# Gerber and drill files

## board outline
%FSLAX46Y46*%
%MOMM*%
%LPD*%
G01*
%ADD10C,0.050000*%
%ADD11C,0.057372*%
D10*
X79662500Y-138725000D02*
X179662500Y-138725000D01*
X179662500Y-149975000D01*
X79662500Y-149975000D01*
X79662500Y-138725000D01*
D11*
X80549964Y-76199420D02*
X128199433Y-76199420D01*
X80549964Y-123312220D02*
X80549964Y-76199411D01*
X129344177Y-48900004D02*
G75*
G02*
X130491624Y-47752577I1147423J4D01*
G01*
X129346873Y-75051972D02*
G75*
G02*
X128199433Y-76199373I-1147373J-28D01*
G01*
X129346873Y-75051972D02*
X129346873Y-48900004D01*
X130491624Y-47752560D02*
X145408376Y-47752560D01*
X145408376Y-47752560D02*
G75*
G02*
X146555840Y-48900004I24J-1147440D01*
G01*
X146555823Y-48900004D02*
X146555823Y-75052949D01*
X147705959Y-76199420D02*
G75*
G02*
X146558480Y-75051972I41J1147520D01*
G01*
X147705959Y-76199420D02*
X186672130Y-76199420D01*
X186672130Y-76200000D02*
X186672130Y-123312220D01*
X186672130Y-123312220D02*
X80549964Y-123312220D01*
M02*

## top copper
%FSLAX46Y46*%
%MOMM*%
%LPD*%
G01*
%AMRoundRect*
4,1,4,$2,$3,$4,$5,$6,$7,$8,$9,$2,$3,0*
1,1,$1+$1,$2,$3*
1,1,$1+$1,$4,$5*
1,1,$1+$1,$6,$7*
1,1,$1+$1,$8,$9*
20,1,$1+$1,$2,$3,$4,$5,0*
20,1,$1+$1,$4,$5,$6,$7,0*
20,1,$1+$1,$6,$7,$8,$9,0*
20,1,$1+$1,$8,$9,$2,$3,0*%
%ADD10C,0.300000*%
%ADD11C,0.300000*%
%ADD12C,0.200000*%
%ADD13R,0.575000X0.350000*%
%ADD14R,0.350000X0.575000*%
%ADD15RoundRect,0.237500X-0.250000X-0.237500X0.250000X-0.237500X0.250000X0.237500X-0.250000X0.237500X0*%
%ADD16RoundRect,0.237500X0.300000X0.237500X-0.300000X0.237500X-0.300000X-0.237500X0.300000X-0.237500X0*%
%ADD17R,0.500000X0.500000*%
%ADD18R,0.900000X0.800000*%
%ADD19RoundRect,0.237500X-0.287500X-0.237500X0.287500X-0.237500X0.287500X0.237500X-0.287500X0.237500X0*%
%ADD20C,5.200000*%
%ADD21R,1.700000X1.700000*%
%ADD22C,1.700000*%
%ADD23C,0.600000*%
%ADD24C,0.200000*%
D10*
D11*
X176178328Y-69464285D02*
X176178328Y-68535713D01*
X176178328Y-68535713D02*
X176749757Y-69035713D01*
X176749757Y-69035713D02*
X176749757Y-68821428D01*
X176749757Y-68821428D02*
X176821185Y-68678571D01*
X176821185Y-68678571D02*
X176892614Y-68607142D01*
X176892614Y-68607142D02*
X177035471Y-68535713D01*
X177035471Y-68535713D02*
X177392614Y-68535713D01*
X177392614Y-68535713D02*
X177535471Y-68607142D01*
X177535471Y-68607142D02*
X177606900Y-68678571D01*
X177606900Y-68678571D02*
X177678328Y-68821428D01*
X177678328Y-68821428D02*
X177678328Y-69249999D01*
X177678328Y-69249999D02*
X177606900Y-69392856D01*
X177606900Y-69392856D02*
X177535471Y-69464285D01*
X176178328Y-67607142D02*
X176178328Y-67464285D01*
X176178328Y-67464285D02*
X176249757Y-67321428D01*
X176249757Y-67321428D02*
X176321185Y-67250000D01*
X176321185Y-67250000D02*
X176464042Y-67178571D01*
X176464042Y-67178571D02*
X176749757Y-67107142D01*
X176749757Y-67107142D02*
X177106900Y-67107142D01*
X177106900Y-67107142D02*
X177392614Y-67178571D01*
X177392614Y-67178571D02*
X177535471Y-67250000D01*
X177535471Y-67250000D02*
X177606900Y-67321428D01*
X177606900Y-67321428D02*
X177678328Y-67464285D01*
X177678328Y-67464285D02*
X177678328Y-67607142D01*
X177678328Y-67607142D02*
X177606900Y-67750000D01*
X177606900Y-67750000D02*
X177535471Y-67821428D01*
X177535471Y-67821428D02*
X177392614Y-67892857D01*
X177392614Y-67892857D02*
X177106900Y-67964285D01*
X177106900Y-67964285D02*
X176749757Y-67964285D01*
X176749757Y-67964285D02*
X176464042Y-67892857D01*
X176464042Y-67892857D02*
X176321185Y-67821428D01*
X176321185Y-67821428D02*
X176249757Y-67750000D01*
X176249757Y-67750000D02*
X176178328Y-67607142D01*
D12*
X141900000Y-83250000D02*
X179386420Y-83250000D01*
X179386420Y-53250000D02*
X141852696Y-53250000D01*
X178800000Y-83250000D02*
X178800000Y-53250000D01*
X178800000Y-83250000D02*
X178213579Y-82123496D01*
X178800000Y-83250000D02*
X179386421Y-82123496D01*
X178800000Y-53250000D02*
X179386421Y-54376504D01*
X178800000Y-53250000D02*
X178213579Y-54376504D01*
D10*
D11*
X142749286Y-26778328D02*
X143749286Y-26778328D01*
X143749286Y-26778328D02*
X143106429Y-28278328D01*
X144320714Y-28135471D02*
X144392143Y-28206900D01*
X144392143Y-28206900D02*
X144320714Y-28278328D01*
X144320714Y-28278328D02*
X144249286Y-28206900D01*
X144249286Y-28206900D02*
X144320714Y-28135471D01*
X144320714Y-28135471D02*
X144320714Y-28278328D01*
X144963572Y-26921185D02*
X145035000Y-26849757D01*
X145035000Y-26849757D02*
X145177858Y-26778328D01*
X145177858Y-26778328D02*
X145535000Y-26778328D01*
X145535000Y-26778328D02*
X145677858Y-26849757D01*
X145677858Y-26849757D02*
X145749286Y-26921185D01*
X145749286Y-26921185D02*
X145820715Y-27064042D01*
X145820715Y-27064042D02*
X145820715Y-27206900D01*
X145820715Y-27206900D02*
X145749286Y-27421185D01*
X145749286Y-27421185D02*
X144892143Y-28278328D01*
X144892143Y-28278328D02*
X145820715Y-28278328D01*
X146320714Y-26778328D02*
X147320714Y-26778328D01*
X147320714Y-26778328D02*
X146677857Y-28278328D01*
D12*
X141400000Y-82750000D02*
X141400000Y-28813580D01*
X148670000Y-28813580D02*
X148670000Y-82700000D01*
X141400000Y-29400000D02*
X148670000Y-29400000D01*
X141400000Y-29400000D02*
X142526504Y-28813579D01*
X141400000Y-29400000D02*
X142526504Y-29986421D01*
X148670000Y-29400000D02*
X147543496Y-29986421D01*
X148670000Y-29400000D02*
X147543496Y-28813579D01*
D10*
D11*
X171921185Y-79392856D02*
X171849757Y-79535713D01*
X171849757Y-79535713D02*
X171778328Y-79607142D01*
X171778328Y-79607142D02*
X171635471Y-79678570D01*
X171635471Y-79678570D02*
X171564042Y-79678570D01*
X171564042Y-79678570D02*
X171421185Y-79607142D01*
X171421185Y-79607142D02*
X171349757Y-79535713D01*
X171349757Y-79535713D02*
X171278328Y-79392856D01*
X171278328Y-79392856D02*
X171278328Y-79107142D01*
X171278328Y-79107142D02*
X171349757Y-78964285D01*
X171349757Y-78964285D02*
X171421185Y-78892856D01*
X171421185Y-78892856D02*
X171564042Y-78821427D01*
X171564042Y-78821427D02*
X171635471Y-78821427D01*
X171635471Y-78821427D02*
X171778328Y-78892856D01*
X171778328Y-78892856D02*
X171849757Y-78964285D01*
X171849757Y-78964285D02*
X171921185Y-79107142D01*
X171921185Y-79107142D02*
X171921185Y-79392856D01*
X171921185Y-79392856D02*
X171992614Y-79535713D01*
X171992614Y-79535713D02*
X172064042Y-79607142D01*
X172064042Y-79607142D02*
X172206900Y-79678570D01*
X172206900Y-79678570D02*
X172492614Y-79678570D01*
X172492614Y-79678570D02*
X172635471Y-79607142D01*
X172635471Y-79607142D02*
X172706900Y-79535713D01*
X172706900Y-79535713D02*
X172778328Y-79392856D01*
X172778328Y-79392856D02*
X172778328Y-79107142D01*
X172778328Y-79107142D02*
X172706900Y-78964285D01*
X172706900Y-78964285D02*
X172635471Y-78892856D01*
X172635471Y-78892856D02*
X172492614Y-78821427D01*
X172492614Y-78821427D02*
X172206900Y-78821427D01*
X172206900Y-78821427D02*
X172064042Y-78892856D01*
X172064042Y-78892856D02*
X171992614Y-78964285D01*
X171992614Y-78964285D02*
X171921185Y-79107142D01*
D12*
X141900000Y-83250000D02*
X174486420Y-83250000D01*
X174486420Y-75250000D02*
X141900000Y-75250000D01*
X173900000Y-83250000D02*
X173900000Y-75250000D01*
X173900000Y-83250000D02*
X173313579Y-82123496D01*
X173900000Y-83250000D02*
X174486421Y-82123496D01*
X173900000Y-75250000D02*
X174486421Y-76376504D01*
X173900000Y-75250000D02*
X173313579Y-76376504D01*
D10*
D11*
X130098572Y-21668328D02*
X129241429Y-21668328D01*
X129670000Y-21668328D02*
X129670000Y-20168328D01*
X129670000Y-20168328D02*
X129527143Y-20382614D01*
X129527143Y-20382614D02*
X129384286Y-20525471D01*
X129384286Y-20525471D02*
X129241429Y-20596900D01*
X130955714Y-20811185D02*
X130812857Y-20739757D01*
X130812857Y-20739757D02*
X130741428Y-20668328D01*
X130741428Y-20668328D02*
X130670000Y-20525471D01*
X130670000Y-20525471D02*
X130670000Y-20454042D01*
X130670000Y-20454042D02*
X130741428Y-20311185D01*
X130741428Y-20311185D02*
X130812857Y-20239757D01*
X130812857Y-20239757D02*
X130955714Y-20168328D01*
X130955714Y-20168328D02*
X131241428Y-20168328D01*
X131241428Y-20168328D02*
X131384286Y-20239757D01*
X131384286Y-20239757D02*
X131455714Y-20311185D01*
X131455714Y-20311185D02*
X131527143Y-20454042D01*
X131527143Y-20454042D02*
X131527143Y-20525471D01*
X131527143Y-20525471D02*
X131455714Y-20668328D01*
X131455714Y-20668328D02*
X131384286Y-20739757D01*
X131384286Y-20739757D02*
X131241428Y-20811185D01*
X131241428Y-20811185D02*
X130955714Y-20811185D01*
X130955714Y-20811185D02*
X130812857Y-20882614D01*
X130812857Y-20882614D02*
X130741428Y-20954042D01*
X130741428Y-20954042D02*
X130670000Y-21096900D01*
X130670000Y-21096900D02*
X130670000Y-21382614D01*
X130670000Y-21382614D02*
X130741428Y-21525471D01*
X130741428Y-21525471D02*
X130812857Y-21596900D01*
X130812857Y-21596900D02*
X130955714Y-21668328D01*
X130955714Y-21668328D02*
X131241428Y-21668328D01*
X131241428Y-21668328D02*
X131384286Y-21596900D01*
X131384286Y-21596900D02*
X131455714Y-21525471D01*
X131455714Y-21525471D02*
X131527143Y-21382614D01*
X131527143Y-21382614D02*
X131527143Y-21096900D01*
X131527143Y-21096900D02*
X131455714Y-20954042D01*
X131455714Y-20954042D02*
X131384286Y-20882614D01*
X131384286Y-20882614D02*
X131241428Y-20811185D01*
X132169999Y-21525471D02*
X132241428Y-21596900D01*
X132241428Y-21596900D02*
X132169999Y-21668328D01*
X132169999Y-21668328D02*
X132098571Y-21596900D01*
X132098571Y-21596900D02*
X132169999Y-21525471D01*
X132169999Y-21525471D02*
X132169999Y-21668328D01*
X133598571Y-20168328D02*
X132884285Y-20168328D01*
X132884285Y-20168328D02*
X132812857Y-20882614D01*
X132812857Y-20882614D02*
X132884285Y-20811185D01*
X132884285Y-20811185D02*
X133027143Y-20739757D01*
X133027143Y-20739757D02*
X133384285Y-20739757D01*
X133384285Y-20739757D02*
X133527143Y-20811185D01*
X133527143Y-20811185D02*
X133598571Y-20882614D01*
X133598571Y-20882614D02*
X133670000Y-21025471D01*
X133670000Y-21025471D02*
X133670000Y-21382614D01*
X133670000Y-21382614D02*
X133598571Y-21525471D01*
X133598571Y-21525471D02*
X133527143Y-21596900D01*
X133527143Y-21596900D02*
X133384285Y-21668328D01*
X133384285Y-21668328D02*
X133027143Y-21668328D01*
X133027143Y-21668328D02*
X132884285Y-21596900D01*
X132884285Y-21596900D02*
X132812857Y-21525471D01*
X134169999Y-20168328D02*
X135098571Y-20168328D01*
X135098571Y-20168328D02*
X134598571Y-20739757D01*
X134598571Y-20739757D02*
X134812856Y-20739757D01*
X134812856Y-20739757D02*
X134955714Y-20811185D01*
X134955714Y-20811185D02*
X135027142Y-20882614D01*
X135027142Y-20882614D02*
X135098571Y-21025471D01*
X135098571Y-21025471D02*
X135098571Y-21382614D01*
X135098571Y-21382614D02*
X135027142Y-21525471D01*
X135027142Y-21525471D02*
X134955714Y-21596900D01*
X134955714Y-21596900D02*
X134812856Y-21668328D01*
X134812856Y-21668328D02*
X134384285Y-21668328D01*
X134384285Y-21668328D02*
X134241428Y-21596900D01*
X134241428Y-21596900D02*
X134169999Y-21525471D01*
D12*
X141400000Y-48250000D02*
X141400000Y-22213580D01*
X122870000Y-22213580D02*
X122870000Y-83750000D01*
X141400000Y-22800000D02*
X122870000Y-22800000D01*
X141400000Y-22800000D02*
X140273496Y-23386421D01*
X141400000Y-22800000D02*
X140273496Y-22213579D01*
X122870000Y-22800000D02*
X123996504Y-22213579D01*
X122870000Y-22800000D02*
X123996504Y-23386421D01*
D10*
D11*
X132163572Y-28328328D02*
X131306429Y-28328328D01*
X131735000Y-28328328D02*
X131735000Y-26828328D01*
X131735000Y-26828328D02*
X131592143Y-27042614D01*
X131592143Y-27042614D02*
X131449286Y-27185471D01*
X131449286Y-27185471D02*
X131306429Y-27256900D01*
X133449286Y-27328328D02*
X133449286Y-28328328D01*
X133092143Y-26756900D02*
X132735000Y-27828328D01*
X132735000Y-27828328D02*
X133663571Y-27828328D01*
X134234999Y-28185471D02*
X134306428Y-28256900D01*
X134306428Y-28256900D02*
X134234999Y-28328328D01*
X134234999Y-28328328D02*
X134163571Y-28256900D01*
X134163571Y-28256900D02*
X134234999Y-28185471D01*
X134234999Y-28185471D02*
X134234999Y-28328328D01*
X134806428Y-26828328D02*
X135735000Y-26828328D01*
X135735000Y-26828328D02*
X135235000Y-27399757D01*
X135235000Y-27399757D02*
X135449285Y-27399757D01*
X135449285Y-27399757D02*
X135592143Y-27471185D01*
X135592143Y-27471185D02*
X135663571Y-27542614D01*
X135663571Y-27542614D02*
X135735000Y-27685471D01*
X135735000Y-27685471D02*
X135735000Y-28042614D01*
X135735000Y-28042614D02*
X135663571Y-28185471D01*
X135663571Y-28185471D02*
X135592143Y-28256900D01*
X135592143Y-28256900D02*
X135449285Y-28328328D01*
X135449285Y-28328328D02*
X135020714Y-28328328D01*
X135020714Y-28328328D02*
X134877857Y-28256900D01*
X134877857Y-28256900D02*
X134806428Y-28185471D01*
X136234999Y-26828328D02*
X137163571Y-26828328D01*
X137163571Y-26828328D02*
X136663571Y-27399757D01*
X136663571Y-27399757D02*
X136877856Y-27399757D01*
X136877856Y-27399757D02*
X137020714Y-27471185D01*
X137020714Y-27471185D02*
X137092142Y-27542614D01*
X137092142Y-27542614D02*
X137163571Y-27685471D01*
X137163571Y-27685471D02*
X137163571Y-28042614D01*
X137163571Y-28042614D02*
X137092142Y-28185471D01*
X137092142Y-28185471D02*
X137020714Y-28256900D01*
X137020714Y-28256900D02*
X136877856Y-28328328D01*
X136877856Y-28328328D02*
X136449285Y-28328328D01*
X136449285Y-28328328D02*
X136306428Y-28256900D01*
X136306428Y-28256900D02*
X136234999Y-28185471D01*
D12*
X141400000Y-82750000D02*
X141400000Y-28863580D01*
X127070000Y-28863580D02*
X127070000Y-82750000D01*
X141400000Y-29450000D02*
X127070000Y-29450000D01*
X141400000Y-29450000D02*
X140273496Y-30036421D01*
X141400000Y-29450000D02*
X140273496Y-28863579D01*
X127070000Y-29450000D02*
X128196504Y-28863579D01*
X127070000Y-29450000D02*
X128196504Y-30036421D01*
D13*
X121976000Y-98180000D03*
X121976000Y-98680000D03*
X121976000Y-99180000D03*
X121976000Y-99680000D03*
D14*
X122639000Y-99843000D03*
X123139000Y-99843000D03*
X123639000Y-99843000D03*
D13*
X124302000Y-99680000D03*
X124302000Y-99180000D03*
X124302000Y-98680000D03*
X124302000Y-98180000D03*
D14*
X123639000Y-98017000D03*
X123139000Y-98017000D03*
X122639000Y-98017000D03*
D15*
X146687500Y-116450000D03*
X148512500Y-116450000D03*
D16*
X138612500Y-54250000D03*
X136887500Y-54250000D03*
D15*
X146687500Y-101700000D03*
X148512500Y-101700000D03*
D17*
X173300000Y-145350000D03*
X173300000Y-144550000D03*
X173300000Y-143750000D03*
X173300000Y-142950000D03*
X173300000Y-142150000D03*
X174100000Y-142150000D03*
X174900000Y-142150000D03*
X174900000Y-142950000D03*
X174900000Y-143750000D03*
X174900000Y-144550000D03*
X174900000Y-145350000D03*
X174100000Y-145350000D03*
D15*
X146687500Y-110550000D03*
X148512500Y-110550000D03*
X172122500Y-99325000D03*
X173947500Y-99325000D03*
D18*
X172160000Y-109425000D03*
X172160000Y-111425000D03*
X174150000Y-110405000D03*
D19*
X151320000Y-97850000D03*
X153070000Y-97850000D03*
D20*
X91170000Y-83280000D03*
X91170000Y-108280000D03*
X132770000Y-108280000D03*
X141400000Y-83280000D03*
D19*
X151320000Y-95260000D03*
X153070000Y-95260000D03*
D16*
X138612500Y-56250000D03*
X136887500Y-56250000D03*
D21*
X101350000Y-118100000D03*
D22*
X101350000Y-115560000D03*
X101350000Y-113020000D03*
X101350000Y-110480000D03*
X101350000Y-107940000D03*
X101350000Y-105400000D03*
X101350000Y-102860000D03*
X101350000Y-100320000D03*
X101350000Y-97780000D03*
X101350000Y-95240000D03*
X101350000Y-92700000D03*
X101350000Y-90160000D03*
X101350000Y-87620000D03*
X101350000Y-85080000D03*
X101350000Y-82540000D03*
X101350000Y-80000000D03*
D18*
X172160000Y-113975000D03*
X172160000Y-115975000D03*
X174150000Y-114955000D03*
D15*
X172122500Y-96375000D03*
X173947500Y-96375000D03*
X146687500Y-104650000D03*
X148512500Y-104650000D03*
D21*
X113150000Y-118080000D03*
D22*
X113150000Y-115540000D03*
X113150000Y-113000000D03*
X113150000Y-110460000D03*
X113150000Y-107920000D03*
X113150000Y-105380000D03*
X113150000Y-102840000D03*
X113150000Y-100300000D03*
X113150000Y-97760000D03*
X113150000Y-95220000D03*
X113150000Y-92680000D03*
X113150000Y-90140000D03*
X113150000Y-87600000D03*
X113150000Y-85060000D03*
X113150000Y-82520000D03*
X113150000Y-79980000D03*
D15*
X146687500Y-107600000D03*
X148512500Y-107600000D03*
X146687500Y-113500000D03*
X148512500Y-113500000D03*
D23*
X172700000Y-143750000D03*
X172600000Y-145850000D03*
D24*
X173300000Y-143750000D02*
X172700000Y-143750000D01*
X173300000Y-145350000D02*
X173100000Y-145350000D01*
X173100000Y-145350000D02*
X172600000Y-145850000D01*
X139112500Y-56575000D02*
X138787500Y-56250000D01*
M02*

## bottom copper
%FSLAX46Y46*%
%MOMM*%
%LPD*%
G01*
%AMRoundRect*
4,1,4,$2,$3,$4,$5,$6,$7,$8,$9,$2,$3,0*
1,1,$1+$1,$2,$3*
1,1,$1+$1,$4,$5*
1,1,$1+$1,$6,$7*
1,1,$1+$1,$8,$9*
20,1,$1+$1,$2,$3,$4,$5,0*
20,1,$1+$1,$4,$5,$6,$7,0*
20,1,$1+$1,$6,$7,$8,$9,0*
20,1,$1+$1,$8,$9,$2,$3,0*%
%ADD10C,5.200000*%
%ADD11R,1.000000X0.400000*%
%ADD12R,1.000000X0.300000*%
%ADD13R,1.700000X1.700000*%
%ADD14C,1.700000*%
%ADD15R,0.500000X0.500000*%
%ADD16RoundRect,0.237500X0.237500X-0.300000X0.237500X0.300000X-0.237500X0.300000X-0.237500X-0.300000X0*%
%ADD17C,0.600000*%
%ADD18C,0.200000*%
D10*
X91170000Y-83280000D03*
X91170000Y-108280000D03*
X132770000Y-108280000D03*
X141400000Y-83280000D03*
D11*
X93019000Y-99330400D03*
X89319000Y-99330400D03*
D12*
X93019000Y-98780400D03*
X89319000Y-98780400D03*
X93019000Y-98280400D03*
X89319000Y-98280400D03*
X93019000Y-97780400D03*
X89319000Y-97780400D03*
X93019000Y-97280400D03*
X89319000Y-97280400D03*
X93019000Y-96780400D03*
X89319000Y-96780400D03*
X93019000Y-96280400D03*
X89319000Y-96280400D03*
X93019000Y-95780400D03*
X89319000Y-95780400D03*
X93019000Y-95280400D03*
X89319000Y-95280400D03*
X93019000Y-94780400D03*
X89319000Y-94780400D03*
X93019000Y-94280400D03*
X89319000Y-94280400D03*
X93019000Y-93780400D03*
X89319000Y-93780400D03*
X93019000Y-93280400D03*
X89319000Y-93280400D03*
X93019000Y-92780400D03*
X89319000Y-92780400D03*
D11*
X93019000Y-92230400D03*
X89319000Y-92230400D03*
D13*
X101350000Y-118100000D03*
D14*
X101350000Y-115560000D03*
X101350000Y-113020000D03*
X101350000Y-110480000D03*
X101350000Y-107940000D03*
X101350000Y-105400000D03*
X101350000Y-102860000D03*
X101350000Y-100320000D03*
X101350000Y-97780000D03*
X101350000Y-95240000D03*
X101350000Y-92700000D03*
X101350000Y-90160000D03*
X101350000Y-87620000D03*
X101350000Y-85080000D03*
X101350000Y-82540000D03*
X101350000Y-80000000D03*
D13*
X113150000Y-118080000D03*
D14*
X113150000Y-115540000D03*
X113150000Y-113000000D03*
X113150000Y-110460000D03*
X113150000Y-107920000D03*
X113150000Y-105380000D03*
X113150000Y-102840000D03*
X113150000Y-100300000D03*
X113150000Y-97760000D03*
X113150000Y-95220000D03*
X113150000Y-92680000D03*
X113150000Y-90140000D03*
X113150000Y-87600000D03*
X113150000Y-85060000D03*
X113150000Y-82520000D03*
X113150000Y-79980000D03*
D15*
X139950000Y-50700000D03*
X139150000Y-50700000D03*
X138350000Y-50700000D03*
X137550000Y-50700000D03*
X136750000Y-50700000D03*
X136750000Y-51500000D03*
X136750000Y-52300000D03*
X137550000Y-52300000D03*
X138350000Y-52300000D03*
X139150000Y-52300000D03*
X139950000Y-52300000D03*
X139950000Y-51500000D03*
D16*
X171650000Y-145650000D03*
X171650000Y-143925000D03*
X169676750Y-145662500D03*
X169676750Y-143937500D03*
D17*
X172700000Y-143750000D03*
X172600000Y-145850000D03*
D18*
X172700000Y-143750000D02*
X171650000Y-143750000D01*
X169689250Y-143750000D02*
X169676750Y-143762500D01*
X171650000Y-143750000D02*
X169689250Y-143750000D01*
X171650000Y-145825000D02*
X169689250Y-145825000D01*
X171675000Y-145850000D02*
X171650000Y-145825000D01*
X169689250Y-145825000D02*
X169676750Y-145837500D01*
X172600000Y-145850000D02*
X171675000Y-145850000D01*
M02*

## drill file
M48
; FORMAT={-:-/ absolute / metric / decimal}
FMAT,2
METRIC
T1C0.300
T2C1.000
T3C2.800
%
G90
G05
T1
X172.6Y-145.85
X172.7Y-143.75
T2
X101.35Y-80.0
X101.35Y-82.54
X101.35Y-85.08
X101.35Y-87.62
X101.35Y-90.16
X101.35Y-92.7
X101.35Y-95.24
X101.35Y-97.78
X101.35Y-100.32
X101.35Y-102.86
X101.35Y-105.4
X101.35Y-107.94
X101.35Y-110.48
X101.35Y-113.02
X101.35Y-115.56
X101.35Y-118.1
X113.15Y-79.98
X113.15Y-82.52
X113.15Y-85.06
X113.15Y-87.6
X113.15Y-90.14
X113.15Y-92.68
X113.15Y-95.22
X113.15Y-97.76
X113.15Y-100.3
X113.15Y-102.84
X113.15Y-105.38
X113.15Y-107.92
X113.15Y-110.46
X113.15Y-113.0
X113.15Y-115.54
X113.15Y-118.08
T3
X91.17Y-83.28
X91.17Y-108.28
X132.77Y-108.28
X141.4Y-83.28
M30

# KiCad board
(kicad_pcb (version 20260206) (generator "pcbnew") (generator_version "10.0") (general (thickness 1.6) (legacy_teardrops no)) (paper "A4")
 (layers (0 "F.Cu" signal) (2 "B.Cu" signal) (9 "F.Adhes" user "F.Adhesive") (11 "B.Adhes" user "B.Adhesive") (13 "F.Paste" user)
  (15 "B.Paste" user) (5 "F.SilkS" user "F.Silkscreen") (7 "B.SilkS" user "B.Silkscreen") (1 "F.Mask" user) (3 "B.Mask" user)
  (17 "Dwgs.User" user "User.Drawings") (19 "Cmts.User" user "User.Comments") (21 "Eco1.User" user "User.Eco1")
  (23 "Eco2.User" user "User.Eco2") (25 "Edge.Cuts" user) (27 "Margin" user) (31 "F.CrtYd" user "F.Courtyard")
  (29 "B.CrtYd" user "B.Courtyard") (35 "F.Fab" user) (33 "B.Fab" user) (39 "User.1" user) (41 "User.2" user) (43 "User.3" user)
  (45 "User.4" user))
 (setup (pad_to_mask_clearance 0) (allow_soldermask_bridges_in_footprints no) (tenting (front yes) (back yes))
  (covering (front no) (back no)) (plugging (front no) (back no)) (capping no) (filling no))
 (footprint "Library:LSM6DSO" (layer "F.Cu") (at 123.139 98.93)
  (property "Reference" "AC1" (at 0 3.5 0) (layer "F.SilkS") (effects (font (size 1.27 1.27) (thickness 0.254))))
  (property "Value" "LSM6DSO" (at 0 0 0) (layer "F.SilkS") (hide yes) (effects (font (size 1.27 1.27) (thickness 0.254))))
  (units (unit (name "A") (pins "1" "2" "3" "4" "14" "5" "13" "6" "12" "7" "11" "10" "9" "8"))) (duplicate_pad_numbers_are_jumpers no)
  (pad "1" smd rect (at -1.163 -0.75 90) (size 0.35 0.575) (layers "F.Cu" "F.Mask" "F.Paste") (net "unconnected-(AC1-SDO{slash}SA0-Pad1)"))
  (pad "2" smd rect (at -1.163 -0.25 90) (size 0.35 0.575) (layers "F.Cu" "F.Mask" "F.Paste") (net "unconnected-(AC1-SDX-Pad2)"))
  (pad "3" smd rect (at -1.163 0.25 90) (size 0.35 0.575) (layers "F.Cu" "F.Mask" "F.Paste") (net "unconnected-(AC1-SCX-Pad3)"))
  (pad "4" smd rect (at -1.163 0.75 90) (size 0.35 0.575) (layers "F.Cu" "F.Mask" "F.Paste") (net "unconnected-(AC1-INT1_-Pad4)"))
  (pad "5" smd rect (at -0.5 0.913) (size 0.35 0.575) (layers "F.Cu" "F.Mask" "F.Paste") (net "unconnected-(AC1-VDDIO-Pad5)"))
  (pad "6" smd rect (at 0 0.913) (size 0.35 0.575) (layers "F.Cu" "F.Mask" "F.Paste") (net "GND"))
  (pad "7" smd rect (at 0.5 0.913) (size 0.35 0.575) (layers "F.Cu" "F.Mask" "F.Paste") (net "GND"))
  (pad "8" smd rect (at 1.163 0.75 90) (size 0.35 0.575) (layers "F.Cu" "F.Mask" "F.Paste") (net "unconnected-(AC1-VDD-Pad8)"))
  (pad "9" smd rect (at 1.163 0.25 90) (size 0.35 0.575) (layers "F.Cu" "F.Mask" "F.Paste") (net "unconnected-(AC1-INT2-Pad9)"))
  (pad "10" smd rect (at 1.163 -0.25 90) (size 0.35 0.575) (layers "F.Cu" "F.Mask" "F.Paste") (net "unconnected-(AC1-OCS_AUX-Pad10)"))
  (pad "11" smd rect (at 1.163 -0.75 90) (size 0.35 0.575) (layers "F.Cu" "F.Mask" "F.Paste") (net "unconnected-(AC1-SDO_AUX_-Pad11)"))
  (pad "12" smd rect (at 0.5 -0.913) (size 0.35 0.575) (layers "F.Cu" "F.Mask" "F.Paste") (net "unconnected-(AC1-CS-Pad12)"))
  (pad "13" smd rect (at 0 -0.913) (size 0.35 0.575) (layers "F.Cu" "F.Mask" "F.Paste") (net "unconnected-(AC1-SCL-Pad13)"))
  (pad "14" smd rect (at -0.5 -0.913) (size 0.35 0.575) (layers "F.Cu" "F.Mask" "F.Paste") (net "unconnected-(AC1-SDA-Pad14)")))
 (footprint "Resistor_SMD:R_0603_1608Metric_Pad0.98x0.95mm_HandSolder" (layer "F.Cu") (at 147.6 116.45)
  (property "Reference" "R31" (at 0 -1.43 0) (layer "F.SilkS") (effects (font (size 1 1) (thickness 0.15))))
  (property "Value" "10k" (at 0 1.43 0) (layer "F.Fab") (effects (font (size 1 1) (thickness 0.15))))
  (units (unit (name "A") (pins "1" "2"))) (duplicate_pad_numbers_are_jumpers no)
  (pad "1" smd roundrect (at -0.9125 0) (size 0.975 0.95) (layers "F.Cu" "F.Mask" "F.Paste") (roundrect_rratio 0.25) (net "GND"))
  (pad "2" smd roundrect (at 0.9125 0) (size 0.975 0.95) (layers "F.Cu" "F.Mask" "F.Paste") (roundrect_rratio 0.25) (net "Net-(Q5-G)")))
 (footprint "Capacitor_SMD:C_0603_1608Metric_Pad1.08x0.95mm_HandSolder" (layer "F.Cu") (at 137.75 54.25 180)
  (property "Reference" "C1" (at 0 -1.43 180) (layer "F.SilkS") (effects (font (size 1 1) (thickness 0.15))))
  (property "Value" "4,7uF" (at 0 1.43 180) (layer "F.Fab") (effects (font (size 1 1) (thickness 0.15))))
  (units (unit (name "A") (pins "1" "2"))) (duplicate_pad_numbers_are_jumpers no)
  (pad "1" smd roundrect (at -0.8625 0 180) (size 1.075 0.95) (layers "F.Cu" "F.Mask" "F.Paste") (roundrect_rratio 0.25) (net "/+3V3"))
  (pad "2" smd roundrect (at 0.8625 0 180) (size 1.075 0.95) (layers "F.Cu" "F.Mask" "F.Paste") (roundrect_rratio 0.25) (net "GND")))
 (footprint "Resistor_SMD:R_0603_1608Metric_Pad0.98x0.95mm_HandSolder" (layer "F.Cu") (at 147.6 101.7)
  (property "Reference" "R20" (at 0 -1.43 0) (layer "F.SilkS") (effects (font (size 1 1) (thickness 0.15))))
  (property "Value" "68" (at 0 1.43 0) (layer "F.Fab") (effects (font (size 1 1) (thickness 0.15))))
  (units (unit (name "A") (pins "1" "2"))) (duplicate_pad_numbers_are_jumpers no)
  (pad "1" smd roundrect (at -0.9125 0) (size 0.975 0.95) (layers "F.Cu" "F.Mask" "F.Paste") (roundrect_rratio 0.25) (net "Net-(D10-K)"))
  (pad "2" smd roundrect (at 0.9125 0) (size 0.975 0.95) (layers "F.Cu" "F.Mask" "F.Paste") (roundrect_rratio 0.25) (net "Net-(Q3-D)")))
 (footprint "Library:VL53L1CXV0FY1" (layer "F.Cu") (at 174.1 143.75 90)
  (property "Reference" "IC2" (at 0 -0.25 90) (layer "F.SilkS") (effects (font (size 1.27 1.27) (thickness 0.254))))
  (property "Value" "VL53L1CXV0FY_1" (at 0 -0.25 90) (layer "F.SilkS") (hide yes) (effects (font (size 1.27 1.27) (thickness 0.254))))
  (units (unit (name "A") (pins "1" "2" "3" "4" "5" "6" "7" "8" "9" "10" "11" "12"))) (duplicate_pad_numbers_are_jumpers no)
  (pad "1" smd rect (at -1.6 -0.8 180) (size 0.5 0.5) (layers "F.Cu" "F.Mask" "F.Paste") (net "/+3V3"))
  (pad "2" smd rect (at -0.8 -0.8 180) (size 0.5 0.5) (layers "F.Cu" "F.Mask" "F.Paste") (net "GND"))
  (pad "3" smd rect (at 0 -0.8 180) (size 0.5 0.5) (layers "F.Cu" "F.Mask" "F.Paste") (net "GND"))
  (pad "4" smd rect (at 0.8 -0.8 180) (size 0.5 0.5) (layers "F.Cu" "F.Mask" "F.Paste") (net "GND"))
  (pad "5" smd rect (at 1.6 -0.8 180) (size 0.5 0.5) (layers "F.Cu" "F.Mask" "F.Paste") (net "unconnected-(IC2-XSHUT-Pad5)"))
  (pad "6" smd rect (at 1.6 0 180) (size 0.5 0.5) (layers "F.Cu" "F.Mask" "F.Paste") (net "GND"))
  (pad "7" smd rect (at 1.6 0.8 180) (size 0.5 0.5) (layers "F.Cu" "F.Mask" "F.Paste") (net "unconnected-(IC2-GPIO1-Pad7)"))
  (pad "8" smd rect (at 0.8 0.8 180) (size 0.5 0.5) (layers "F.Cu" "F.Mask" "F.Paste") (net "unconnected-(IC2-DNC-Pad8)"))
  (pad "9" smd rect (at 0 0.8 180) (size 0.5 0.5) (layers "F.Cu" "F.Mask" "F.Paste") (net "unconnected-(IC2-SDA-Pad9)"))
  (pad "10" smd rect (at -0.8 0.8 180) (size 0.5 0.5) (layers "F.Cu" "F.Mask" "F.Paste") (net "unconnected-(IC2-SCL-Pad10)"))
  (pad "11" smd rect (at -1.6 0.8 180) (size 0.5 0.5) (layers "F.Cu" "F.Mask" "F.Paste") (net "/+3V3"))
  (pad "12" smd rect (at -1.6 0 180) (size 0.5 0.5) (layers "F.Cu" "F.Mask" "F.Paste") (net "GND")))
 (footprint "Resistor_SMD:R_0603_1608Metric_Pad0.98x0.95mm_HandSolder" (layer "F.Cu") (at 147.6 110.55)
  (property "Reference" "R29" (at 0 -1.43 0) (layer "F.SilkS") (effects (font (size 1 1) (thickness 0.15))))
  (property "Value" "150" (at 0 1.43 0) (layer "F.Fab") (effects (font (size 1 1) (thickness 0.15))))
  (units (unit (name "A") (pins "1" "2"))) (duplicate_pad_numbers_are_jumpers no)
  (pad "1" smd roundrect (at -0.9125 0) (size 0.975 0.95) (layers "F.Cu" "F.Mask" "F.Paste") (roundrect_rratio 0.25) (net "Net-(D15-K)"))
  (pad "2" smd roundrect (at 0.9125 0) (size 0.975 0.95) (layers "F.Cu" "F.Mask" "F.Paste") (roundrect_rratio 0.25) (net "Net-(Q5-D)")))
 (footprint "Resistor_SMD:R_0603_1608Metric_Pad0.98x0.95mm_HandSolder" (layer "F.Cu") (at 173.035 99.325)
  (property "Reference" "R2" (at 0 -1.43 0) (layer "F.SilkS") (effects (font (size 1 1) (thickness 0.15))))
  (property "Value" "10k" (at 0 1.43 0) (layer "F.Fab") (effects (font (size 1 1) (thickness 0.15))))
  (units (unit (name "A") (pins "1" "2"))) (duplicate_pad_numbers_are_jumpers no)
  (pad "1" smd roundrect (at -0.9125 0) (size 0.975 0.95) (layers "F.Cu" "F.Mask" "F.Paste") (roundrect_rratio 0.25)
   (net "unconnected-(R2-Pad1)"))
  (pad "2" smd roundrect (at 0.9125 0) (size 0.975 0.95) (layers "F.Cu" "F.Mask" "F.Paste") (roundrect_rratio 0.25)
   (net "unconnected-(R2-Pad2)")))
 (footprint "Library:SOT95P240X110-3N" (layer "F.Cu") (at 173.15 110.425)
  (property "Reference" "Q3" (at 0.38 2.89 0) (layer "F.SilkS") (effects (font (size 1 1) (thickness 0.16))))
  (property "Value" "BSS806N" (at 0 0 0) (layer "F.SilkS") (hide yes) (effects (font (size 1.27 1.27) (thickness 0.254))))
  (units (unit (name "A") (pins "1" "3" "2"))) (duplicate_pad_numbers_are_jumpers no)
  (pad "1" smd rect (at -0.99 -1) (size 0.9 0.8) (layers "F.Cu" "F.Mask" "F.Paste") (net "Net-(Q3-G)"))
  (pad "2" smd rect (at -0.99 1) (size 0.9 0.8) (layers "F.Cu" "F.Mask" "F.Paste") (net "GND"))
  (pad "3" smd rect (at 1 -0.02) (size 0.9 0.8) (layers "F.Cu" "F.Mask" "F.Paste") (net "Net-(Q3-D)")))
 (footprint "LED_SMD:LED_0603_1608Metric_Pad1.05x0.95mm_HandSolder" (layer "F.Cu") (at 152.195 97.85)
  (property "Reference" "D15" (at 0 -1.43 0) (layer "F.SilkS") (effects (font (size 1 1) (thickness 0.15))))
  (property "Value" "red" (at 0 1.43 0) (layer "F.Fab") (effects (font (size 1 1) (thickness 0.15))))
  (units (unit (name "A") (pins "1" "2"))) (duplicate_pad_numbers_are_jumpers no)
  (pad "1" smd roundrect (at -0.875 0) (size 1.05 0.95) (layers "F.Cu" "F.Mask" "F.Paste") (roundrect_rratio 0.25) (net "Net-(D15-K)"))
  (pad "2" smd roundrect (at 0.875 0) (size 1.05 0.95) (layers "F.Cu" "F.Mask" "F.Paste") (roundrect_rratio 0.25) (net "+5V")))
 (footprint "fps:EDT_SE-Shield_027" (layer "F.Cu") (at 91.17 108.28)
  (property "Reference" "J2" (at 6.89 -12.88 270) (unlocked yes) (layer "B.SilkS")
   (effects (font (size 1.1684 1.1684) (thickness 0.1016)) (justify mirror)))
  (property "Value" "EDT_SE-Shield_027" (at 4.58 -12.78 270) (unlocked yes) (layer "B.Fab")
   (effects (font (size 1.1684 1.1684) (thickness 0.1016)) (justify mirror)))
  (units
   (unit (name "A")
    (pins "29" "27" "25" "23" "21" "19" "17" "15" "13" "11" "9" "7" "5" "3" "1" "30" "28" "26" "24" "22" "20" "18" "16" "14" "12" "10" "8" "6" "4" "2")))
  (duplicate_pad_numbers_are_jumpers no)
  (pad "" thru_hole circle (at 0 -25) (size 5.2 5.2) (drill 2.8) (layers "*.Cu" "*.Mask") (remove_unused_layers no))
  (pad "" thru_hole circle (at 0 0) (size 5.2 5.2) (drill 2.8) (layers "*.Cu" "*.Mask") (remove_unused_layers no))
  (pad "" thru_hole circle (at 41.6 0) (size 5.2 5.2) (drill 2.8) (layers "*.Cu" "*.Mask") (remove_unused_layers no))
  (pad "" thru_hole circle (at 50.23 -25) (size 5.2 5.2) (drill 2.8) (layers "*.Cu" "*.Mask") (remove_unused_layers no))
  (pad "1" smd rect (at 1.849 -8.9496 180) (size 1 0.4) (layers "B.Cu" "B.Mask" "B.Paste") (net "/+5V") (solder_mask_margin 0.075)
   (solder_paste_margin 0) (thermal_bridge_angle 0))
  (pad "2" smd rect (at -1.851 -8.9496 180) (size 1 0.4) (layers "B.Cu" "B.Mask" "B.Paste") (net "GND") (solder_mask_margin 0.075)
   (solder_paste_margin 0) (thermal_bridge_angle 0))
  (pad "3" smd rect (at 1.849 -9.4996 180) (size 1 0.3) (layers "B.Cu" "B.Mask" "B.Paste") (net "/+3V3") (solder_mask_margin 0.075)
   (solder_paste_margin 0) (thermal_bridge_angle 0))
  (pad "4" smd rect (at -1.851 -9.4996 180) (size 1 0.3) (layers "B.Cu" "B.Mask" "B.Paste") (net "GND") (solder_mask_margin 0.075)
   (solder_paste_margin 0) (thermal_bridge_angle 0))
  (pad "5" smd rect (at 1.849 -9.9996 180) (size 1 0.3) (layers "B.Cu" "B.Mask" "B.Paste") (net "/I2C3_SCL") (solder_mask_margin 0.075)
   (solder_paste_margin 0) (thermal_bridge_angle 0))
  (pad "6" smd rect (at -1.851 -9.9996 180) (size 1 0.3) (layers "B.Cu" "B.Mask" "B.Paste") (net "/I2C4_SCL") (solder_mask_margin 0.075)
   (solder_paste_margin 0) (thermal_bridge_angle 0))
  (pad "7" smd rect (at 1.849 -10.4996 180) (size 1 0.3) (layers "B.Cu" "B.Mask" "B.Paste") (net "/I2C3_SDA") (solder_mask_margin 0.075)
   (solder_paste_margin 0) (thermal_bridge_angle 0))
  (pad "8" smd rect (at -1.851 -10.4996 180) (size 1 0.3) (layers "B.Cu" "B.Mask" "B.Paste") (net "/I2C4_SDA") (solder_mask_margin 0.075)
   (solder_paste_margin 0) (thermal_bridge_angle 0))
  (pad "9" smd rect (at 1.849 -10.9996 180) (size 1 0.3) (layers "B.Cu" "B.Mask" "B.Paste") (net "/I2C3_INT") (solder_mask_margin 0.075)
   (solder_paste_margin 0) (thermal_bridge_angle 0))
  (pad "10" smd rect (at -1.851 -10.9996 180) (size 1 0.3) (layers "B.Cu" "B.Mask" "B.Paste") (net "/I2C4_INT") (solder_mask_margin 0.075)
   (solder_paste_margin 0) (thermal_bridge_angle 0))
  (pad "11" smd rect (at 1.849 -11.4996 180) (size 1 0.3) (layers "B.Cu" "B.Mask" "B.Paste") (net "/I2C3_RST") (solder_mask_margin 0.075)
   (solder_paste_margin 0) (thermal_bridge_angle 0))
  (pad "12" smd rect (at -1.851 -11.4996 180) (size 1 0.3) (layers "B.Cu" "B.Mask" "B.Paste") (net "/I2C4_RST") (solder_mask_margin 0.075)
   (solder_paste_margin 0) (thermal_bridge_angle 0))
  (pad "13" smd rect (at 1.849 -11.9996 180) (size 1 0.3) (layers "B.Cu" "B.Mask" "B.Paste") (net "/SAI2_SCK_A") (solder_mask_margin 0.075)
   (solder_paste_margin 0) (thermal_bridge_angle 0))
  (pad "14" smd rect (at -1.851 -11.9996 180) (size 1 0.3) (layers "B.Cu" "B.Mask" "B.Paste") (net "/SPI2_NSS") (solder_mask_margin 0.075)
   (solder_paste_margin 0) (thermal_bridge_angle 0))
  (pad "15" smd rect (at 1.849 -12.4996 180) (size 1 0.3) (layers "B.Cu" "B.Mask" "B.Paste") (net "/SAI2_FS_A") (solder_mask_margin 0.075)
   (solder_paste_margin 0) (thermal_bridge_angle 0))
  (pad "16" smd rect (at -1.851 -12.4996 180) (size 1 0.3) (layers "B.Cu" "B.Mask" "B.Paste") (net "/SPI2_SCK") (solder_mask_margin 0.075)
   (solder_paste_margin 0) (thermal_bridge_angle 0))
  (pad "17" smd rect (at 1.849 -12.9996 180) (size 1 0.3) (layers "B.Cu" "B.Mask" "B.Paste") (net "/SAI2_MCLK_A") (solder_mask_margin 0.075)
   (solder_paste_margin 0) (thermal_bridge_angle 0))
  (pad "18" smd rect (at -1.851 -12.9996 180) (size 1 0.3) (layers "B.Cu" "B.Mask" "B.Paste") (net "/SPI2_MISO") (solder_mask_margin 0.075)
   (solder_paste_margin 0) (thermal_bridge_angle 0))
  (pad "19" smd rect (at 1.849 -13.4996 180) (size 1 0.3) (layers "B.Cu" "B.Mask" "B.Paste") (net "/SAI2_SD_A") (solder_mask_margin 0.075)
   (solder_paste_margin 0) (thermal_bridge_angle 0))
  (pad "20" smd rect (at -1.851 -13.4996 180) (size 1 0.3) (layers "B.Cu" "B.Mask" "B.Paste") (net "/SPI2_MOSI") (solder_mask_margin 0.075)
   (solder_paste_margin 0) (thermal_bridge_angle 0))
  (pad "21" smd rect (at 1.849 -13.9996 180) (size 1 0.3) (layers "B.Cu" "B.Mask" "B.Paste") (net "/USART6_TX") (solder_mask_margin 0.075)
   (solder_paste_margin 0) (thermal_bridge_angle 0))
  (pad "22" smd rect (at -1.851 -13.9996 180) (size 1 0.3) (layers "B.Cu" "B.Mask" "B.Paste") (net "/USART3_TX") (solder_mask_margin 0.075)
   (solder_paste_margin 0) (thermal_bridge_angle 0))
  (pad "23" smd rect (at 1.849 -14.4996 180) (size 1 0.3) (layers "B.Cu" "B.Mask" "B.Paste") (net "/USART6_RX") (solder_mask_margin 0.075)
   (solder_paste_margin 0) (thermal_bridge_angle 0))
  (pad "24" smd rect (at -1.851 -14.4996 180) (size 1 0.3) (layers "B.Cu" "B.Mask" "B.Paste") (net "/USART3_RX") (solder_mask_margin 0.075)
   (solder_paste_margin 0) (thermal_bridge_angle 0))
  (pad "25" smd rect (at 1.849 -14.9996 180) (size 1 0.3) (layers "B.Cu" "B.Mask" "B.Paste") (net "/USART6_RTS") (solder_mask_margin 0.075)
   (solder_paste_margin 0) (thermal_bridge_angle 0))
  (pad "26" smd rect (at -1.851 -14.9996 180) (size 1 0.3) (layers "B.Cu" "B.Mask" "B.Paste") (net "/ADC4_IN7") (solder_mask_margin 0.075)
   (solder_paste_margin 0) (thermal_bridge_angle 0))
  (pad "27" smd rect (at 1.849 -15.4996 180) (size 1 0.3) (layers "B.Cu" "B.Mask" "B.Paste") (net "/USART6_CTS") (solder_mask_margin 0.075)
   (solder_paste_margin 0) (thermal_bridge_angle 0))
  (pad "28" smd rect (at -1.851 -15.4996 180) (size 1 0.3) (layers "B.Cu" "B.Mask" "B.Paste") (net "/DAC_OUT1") (solder_mask_margin 0.075)
   (solder_paste_margin 0) (thermal_bridge_angle 0))
  (pad "29" smd rect (at 1.849 -16.0496 180) (size 1 0.4) (layers "B.Cu" "B.Mask" "B.Paste") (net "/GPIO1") (solder_mask_margin 0.075)
   (solder_paste_margin 0) (thermal_bridge_angle 0))
  (pad "30" smd rect (at -1.851 -16.0496 180) (size 1 0.4) (layers "B.Cu" "B.Mask" "B.Paste") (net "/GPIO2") (solder_mask_margin 0.075)
   (solder_paste_margin 0) (thermal_bridge_angle 0)))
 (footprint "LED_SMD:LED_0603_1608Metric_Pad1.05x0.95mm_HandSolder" (layer "F.Cu") (at 152.195 95.26)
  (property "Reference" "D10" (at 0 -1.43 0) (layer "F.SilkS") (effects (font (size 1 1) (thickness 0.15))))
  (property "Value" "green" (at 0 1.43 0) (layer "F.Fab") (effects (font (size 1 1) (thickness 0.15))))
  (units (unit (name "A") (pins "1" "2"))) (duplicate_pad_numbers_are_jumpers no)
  (pad "1" smd roundrect (at -0.875 0) (size 1.05 0.95) (layers "F.Cu" "F.Mask" "F.Paste") (roundrect_rratio 0.25) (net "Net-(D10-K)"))
  (pad "2" smd roundrect (at 0.875 0) (size 1.05 0.95) (layers "F.Cu" "F.Mask" "F.Paste") (roundrect_rratio 0.25) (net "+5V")))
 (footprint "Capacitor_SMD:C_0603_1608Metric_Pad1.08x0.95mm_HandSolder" (layer "F.Cu") (at 137.75 56.25 180)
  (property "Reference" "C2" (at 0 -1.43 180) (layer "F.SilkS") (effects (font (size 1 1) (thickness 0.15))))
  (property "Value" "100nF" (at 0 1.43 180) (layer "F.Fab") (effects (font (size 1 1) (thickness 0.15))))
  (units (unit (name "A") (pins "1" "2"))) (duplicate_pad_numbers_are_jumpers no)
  (pad "1" smd roundrect (at -0.8625 0 180) (size 1.075 0.95) (layers "F.Cu" "F.Mask" "F.Paste") (roundrect_rratio 0.25) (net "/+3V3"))
  (pad "2" smd roundrect (at 0.8625 0 180) (size 1.075 0.95) (layers "F.Cu" "F.Mask" "F.Paste") (roundrect_rratio 0.25) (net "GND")))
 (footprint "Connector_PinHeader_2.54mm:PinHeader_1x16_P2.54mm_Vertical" (layer "F.Cu") (at 101.35 118.1 180)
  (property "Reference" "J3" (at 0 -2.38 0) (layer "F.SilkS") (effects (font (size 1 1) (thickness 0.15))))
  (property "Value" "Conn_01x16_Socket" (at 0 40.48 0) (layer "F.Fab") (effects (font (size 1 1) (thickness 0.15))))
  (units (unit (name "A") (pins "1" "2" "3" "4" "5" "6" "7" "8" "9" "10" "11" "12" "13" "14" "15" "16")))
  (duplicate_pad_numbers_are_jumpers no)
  (pad "1" thru_hole rect (at 0 0 180) (size 1.7 1.7) (drill 1) (layers "*.Cu" "*.Mask") (remove_unused_layers no) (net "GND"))
  (pad "2" thru_hole circle (at 0 2.54 180) (size 1.7 1.7) (drill 1) (layers "*.Cu" "*.Mask") (remove_unused_layers no) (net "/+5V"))
  (pad "3" thru_hole circle (at 0 5.08 180) (size 1.7 1.7) (drill 1) (layers "*.Cu" "*.Mask") (remove_unused_layers no) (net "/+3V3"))
  (pad "4" thru_hole circle (at 0 7.62 180) (size 1.7 1.7) (drill 1) (layers "*.Cu" "*.Mask") (remove_unused_layers no) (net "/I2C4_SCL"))
  (pad "5" thru_hole circle (at 0 10.16 180) (size 1.7 1.7) (drill 1) (layers "*.Cu" "*.Mask") (remove_unused_layers no) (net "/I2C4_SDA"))
  (pad "6" thru_hole circle (at 0 12.7 180) (size 1.7 1.7) (drill 1) (layers "*.Cu" "*.Mask") (remove_unused_layers no) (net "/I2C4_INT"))
  (pad "7" thru_hole circle (at 0 15.24 180) (size 1.7 1.7) (drill 1) (layers "*.Cu" "*.Mask") (remove_unused_layers no) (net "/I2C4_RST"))
  (pad "8" thru_hole circle (at 0 17.78 180) (size 1.7 1.7) (drill 1) (layers "*.Cu" "*.Mask") (remove_unused_layers no) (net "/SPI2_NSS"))
  (pad "9" thru_hole circle (at 0 20.32 180) (size 1.7 1.7) (drill 1) (layers "*.Cu" "*.Mask") (remove_unused_layers no) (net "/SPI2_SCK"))
  (pad "10" thru_hole circle (at 0 22.86 180) (size 1.7 1.7) (drill 1) (layers "*.Cu" "*.Mask") (remove_unused_layers no) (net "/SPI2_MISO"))
  (pad "11" thru_hole circle (at 0 25.4 180) (size 1.7 1.7) (drill 1) (layers "*.Cu" "*.Mask") (remove_unused_layers no) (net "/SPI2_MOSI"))
  (pad "12" thru_hole circle (at 0 27.94 180) (size 1.7 1.7) (drill 1) (layers "*.Cu" "*.Mask") (remove_unused_layers no) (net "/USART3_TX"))
  (pad "13" thru_hole circle (at 0 30.48 180) (size 1.7 1.7) (drill 1) (layers "*.Cu" "*.Mask") (remove_unused_layers no) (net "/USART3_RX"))
  (pad "14" thru_hole circle (at 0 33.02 180) (size 1.7 1.7) (drill 1) (layers "*.Cu" "*.Mask") (remove_unused_layers no) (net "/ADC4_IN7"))
  (pad "15" thru_hole circle (at 0 35.56 180) (size 1.7 1.7) (drill 1) (layers "*.Cu" "*.Mask") (remove_unused_layers no) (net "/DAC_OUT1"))
  (pad "16" thru_hole circle (at 0 38.1 180) (size 1.7 1.7) (drill 1) (layers "*.Cu" "*.Mask") (remove_unused_layers no) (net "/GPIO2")))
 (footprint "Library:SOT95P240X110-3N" (layer "F.Cu") (at 173.15 114.975)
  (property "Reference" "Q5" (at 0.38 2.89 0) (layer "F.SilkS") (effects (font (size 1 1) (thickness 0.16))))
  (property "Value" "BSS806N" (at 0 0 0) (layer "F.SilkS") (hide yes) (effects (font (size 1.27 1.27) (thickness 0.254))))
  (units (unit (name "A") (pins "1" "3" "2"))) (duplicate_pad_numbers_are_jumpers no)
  (pad "1" smd rect (at -0.99 -1) (size 0.9 0.8) (layers "F.Cu" "F.Mask" "F.Paste") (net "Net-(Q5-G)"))
  (pad "2" smd rect (at -0.99 1) (size 0.9 0.8) (layers "F.Cu" "F.Mask" "F.Paste") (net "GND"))
  (pad "3" smd rect (at 1 -0.02) (size 0.9 0.8) (layers "F.Cu" "F.Mask" "F.Paste") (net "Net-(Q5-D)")))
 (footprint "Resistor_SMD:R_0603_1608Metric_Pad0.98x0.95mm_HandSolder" (layer "F.Cu") (at 173.035 96.375)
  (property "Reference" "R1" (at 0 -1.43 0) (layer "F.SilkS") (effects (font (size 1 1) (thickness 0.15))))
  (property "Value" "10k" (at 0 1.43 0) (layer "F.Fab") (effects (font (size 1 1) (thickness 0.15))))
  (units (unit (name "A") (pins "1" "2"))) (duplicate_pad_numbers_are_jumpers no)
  (pad "1" smd roundrect (at -0.9125 0) (size 0.975 0.95) (layers "F.Cu" "F.Mask" "F.Paste") (roundrect_rratio 0.25)
   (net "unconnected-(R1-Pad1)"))
  (pad "2" smd roundrect (at 0.9125 0) (size 0.975 0.95) (layers "F.Cu" "F.Mask" "F.Paste") (roundrect_rratio 0.25)
   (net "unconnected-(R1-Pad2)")))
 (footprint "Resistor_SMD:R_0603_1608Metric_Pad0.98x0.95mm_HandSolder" (layer "F.Cu") (at 147.6 104.65)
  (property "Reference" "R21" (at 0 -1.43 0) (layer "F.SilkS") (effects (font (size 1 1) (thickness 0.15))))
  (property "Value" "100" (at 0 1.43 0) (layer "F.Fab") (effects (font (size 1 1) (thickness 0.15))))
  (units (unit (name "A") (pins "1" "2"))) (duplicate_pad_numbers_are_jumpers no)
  (pad "1" smd roundrect (at -0.9125 0) (size 0.975 0.95) (layers "F.Cu" "F.Mask" "F.Paste") (roundrect_rratio 0.25) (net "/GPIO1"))
  (pad "2" smd roundrect (at 0.9125 0) (size 0.975 0.95) (layers "F.Cu" "F.Mask" "F.Paste") (roundrect_rratio 0.25) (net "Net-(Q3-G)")))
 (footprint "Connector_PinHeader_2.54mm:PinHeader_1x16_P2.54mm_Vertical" (layer "F.Cu") (at 113.15 118.08 180)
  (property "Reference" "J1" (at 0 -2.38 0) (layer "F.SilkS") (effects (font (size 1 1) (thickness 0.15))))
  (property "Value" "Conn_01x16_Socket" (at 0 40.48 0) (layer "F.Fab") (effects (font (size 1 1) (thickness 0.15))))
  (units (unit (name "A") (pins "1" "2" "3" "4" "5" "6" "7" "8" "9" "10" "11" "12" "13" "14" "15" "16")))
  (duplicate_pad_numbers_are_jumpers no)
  (pad "1" thru_hole rect (at 0 0 180) (size 1.7 1.7) (drill 1) (layers "*.Cu" "*.Mask") (remove_unused_layers no) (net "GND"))
  (pad "2" thru_hole circle (at 0 2.54 180) (size 1.7 1.7) (drill 1) (layers "*.Cu" "*.Mask") (remove_unused_layers no) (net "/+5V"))
  (pad "3" thru_hole circle (at 0 5.08 180) (size 1.7 1.7) (drill 1) (layers "*.Cu" "*.Mask") (remove_unused_layers no) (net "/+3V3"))
  (pad "4" thru_hole circle (at 0 7.62 180) (size 1.7 1.7) (drill 1) (layers "*.Cu" "*.Mask") (remove_unused_layers no) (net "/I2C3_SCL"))
  (pad "5" thru_hole circle (at 0 10.16 180) (size 1.7 1.7) (drill 1) (layers "*.Cu" "*.Mask") (remove_unused_layers no) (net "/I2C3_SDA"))
  (pad "6" thru_hole circle (at 0 12.7 180) (size 1.7 1.7) (drill 1) (layers "*.Cu" "*.Mask") (remove_unused_layers no) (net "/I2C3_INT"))
  (pad "7" thru_hole circle (at 0 15.24 180) (size 1.7 1.7) (drill 1) (layers "*.Cu" "*.Mask") (remove_unused_layers no) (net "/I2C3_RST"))
  (pad "8" thru_hole circle (at 0 17.78 180) (size 1.7 1.7) (drill 1) (layers "*.Cu" "*.Mask") (remove_unused_layers no) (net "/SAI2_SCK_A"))
  (pad "9" thru_hole circle (at 0 20.32 180) (size 1.7 1.7) (drill 1) (layers "*.Cu" "*.Mask") (remove_unused_layers no) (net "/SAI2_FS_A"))
  (pad "10" thru_hole circle (at 0 22.86 180) (size 1.7 1.7) (drill 1) (layers "*.Cu" "*.Mask") (remove_unused_layers no)
   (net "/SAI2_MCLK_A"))
  (pad "11" thru_hole circle (at 0 25.4 180) (size 1.7 1.7) (drill 1) (layers "*.Cu" "*.Mask") (remove_unused_layers no) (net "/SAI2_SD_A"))
  (pad "12" thru_hole circle (at 0 27.94 180) (size 1.7 1.7) (drill 1) (layers "*.Cu" "*.Mask") (remove_unused_layers no) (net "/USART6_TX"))
  (pad "13" thru_hole circle (at 0 30.48 180) (size 1.7 1.7) (drill 1) (layers "*.Cu" "*.Mask") (remove_unused_layers no) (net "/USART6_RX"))
  (pad "14" thru_hole circle (at 0 33.02 180) (size 1.7 1.7) (drill 1) (layers "*.Cu" "*.Mask") (remove_unused_layers no)
   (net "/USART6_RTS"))
  (pad "15" thru_hole circle (at 0 35.56 180) (size 1.7 1.7) (drill 1) (layers "*.Cu" "*.Mask") (remove_unused_layers no)
   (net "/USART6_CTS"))
  (pad "16" thru_hole circle (at 0 38.1 180) (size 1.7 1.7) (drill 1) (layers "*.Cu" "*.Mask") (remove_unused_layers no) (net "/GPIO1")))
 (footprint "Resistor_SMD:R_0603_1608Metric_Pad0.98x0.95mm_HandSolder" (layer "F.Cu") (at 147.6 107.6)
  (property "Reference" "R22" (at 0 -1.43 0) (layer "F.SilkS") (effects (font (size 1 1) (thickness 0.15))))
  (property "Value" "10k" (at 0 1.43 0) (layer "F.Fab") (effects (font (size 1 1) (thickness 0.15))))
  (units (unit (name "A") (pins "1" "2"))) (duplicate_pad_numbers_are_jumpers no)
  (pad "1" smd roundrect (at -0.9125 0) (size 0.975 0.95) (layers "F.Cu" "F.Mask" "F.Paste") (roundrect_rratio 0.25) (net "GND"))
  (pad "2" smd roundrect (at 0.9125 0) (size 0.975 0.95) (layers "F.Cu" "F.Mask" "F.Paste") (roundrect_rratio 0.25) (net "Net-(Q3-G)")))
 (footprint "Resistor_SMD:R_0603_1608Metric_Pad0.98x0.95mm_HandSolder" (layer "F.Cu") (at 147.6 113.5)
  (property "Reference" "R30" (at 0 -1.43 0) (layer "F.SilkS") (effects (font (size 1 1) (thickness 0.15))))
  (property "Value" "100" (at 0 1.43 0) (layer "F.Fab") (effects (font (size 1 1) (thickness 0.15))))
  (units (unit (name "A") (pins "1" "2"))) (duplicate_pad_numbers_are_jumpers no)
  (pad "1" smd roundrect (at -0.9125 0) (size 0.975 0.95) (layers "F.Cu" "F.Mask" "F.Paste") (roundrect_rratio 0.25) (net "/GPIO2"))
  (pad "2" smd roundrect (at 0.9125 0) (size 0.975 0.95) (layers "F.Cu" "F.Mask" "F.Paste") (roundrect_rratio 0.25) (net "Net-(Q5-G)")))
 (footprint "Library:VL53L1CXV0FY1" (layer "B.Cu") (at 138.35 51.5 180)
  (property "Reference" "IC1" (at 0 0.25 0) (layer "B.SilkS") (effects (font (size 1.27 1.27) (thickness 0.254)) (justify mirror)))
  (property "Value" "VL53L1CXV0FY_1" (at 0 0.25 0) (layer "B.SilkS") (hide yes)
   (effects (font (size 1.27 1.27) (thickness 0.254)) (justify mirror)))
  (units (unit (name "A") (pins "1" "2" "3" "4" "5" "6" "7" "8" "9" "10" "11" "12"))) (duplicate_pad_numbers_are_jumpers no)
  (pad "1" smd rect (at -1.6 0.8 90) (size 0.5 0.5) (layers "B.Cu" "B.Mask" "B.Paste") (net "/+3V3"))
  (pad "2" smd rect (at -0.8 0.8 90) (size 0.5 0.5) (layers "B.Cu" "B.Mask" "B.Paste") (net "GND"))
  (pad "3" smd rect (at 0 0.8 90) (size 0.5 0.5) (layers "B.Cu" "B.Mask" "B.Paste") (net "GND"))
  (pad "4" smd rect (at 0.8 0.8 90) (size 0.5 0.5) (layers "B.Cu" "B.Mask" "B.Paste") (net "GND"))
  (pad "5" smd rect (at 1.6 0.8 90) (size 0.5 0.5) (layers "B.Cu" "B.Mask" "B.Paste") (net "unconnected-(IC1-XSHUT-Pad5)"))
  (pad "6" smd rect (at 1.6 0 90) (size 0.5 0.5) (layers "B.Cu" "B.Mask" "B.Paste") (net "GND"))
  (pad "7" smd rect (at 1.6 -0.8 90) (size 0.5 0.5) (layers "B.Cu" "B.Mask" "B.Paste") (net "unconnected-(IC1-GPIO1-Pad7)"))
  (pad "8" smd rect (at 0.8 -0.8 90) (size 0.5 0.5) (layers "B.Cu" "B.Mask" "B.Paste") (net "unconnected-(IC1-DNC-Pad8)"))
  (pad "9" smd rect (at 0 -0.8 90) (size 0.5 0.5) (layers "B.Cu" "B.Mask" "B.Paste") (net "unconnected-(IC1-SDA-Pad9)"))
  (pad "10" smd rect (at -0.8 -0.8 90) (size 0.5 0.5) (layers "B.Cu" "B.Mask" "B.Paste") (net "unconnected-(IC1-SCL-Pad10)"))
  (pad "11" smd rect (at -1.6 -0.8 90) (size 0.5 0.5) (layers "B.Cu" "B.Mask" "B.Paste") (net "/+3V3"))
  (pad "12" smd rect (at -1.6 0 90) (size 0.5 0.5) (layers "B.Cu" "B.Mask" "B.Paste") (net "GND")))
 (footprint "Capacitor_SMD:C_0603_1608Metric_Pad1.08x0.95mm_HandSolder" (layer "B.Cu") (at 171.65 144.7875 90)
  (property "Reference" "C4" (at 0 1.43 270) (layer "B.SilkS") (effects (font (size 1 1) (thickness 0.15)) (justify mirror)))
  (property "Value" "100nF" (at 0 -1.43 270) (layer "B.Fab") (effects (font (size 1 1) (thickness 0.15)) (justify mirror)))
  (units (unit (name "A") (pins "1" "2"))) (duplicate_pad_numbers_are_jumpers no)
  (pad "1" smd roundrect (at -0.8625 0 90) (size 1.075 0.95) (layers "B.Cu" "B.Mask" "B.Paste") (roundrect_rratio 0.25) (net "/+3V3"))
  (pad "2" smd roundrect (at 0.8625 0 90) (size 1.075 0.95) (layers "B.Cu" "B.Mask" "B.Paste") (roundrect_rratio 0.25) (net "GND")))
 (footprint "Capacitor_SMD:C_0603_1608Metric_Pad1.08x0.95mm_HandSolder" (layer "B.Cu") (at 169.67675 144.8 90)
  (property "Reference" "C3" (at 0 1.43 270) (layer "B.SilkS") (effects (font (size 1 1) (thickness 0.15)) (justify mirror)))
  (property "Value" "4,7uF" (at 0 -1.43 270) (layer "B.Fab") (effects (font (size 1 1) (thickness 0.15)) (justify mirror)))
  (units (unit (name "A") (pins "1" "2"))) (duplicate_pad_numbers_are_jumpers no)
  (pad "1" smd roundrect (at -0.8625 0 90) (size 1.075 0.95) (layers "B.Cu" "B.Mask" "B.Paste") (roundrect_rratio 0.25) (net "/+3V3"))
  (pad "2" smd roundrect (at 0.8625 0 90) (size 1.075 0.95) (layers "B.Cu" "B.Mask" "B.Paste") (roundrect_rratio 0.25) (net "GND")))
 (gr_rect (start 79.6625 138.725) (end 179.6625 149.975) (stroke (width 0.05) (type solid)) (fill no) (layer "Edge.Cuts"))
 (gr_line (start 80.549964 76.19942) (end 128.199433 76.19942) (stroke (width 0.057372) (type default)) (layer "Edge.Cuts"))
 (gr_line (start 80.549964 123.31222) (end 80.549964 76.199411) (stroke (width 0.057372) (type solid)) (layer "Edge.Cuts"))
 (gr_arc (start 129.344177 48.900004) (mid 129.680249 48.088629) (end 130.491624 47.75256) (stroke (width 0.057372) (type default))
  (layer "Edge.Cuts"))
 (gr_arc (start 129.346873 75.051972) (mid 129.010808 75.863366) (end 128.199433 76.19942) (stroke (width 0.057372) (type default))
  (layer "Edge.Cuts"))
 (gr_line (start 129.346873 75.051972) (end 129.346873 48.900004) (stroke (width 0.057372) (type solid)) (layer "Edge.Cuts"))
 (gr_line (start 130.491624 47.75256) (end 145.408376 47.75256) (stroke (width 0.057372) (type default)) (layer "Edge.Cuts"))
 (gr_arc (start 145.408376 47.75256) (mid 146.219748 48.088632) (end 146.555823 48.900004) (stroke (width 0.057372) (type default))
  (layer "Edge.Cuts"))
 (gr_line (start 146.555823 48.900004) (end 146.555823 75.052949) (stroke (width 0.057372) (type solid)) (layer "Edge.Cuts"))
 (gr_arc (start 147.705959 76.19942) (mid 146.894625 75.863325) (end 146.558519 75.051972) (stroke (width 0.057372) (type default))
  (layer "Edge.Cuts"))
 (gr_line (start 147.705959 76.19942) (end 186.67213 76.19942) (stroke (width 0.057372) (type solid)) (layer "Edge.Cuts"))
 (gr_line (start 186.67213 76.2) (end 186.67213 123.31222) (stroke (width 0.057372) (type solid)) (layer "Edge.Cuts"))
 (gr_line (start 186.67213 123.31222) (end 80.549964 123.31222) (stroke (width 0.057372) (type solid)) (layer "Edge.Cuts"))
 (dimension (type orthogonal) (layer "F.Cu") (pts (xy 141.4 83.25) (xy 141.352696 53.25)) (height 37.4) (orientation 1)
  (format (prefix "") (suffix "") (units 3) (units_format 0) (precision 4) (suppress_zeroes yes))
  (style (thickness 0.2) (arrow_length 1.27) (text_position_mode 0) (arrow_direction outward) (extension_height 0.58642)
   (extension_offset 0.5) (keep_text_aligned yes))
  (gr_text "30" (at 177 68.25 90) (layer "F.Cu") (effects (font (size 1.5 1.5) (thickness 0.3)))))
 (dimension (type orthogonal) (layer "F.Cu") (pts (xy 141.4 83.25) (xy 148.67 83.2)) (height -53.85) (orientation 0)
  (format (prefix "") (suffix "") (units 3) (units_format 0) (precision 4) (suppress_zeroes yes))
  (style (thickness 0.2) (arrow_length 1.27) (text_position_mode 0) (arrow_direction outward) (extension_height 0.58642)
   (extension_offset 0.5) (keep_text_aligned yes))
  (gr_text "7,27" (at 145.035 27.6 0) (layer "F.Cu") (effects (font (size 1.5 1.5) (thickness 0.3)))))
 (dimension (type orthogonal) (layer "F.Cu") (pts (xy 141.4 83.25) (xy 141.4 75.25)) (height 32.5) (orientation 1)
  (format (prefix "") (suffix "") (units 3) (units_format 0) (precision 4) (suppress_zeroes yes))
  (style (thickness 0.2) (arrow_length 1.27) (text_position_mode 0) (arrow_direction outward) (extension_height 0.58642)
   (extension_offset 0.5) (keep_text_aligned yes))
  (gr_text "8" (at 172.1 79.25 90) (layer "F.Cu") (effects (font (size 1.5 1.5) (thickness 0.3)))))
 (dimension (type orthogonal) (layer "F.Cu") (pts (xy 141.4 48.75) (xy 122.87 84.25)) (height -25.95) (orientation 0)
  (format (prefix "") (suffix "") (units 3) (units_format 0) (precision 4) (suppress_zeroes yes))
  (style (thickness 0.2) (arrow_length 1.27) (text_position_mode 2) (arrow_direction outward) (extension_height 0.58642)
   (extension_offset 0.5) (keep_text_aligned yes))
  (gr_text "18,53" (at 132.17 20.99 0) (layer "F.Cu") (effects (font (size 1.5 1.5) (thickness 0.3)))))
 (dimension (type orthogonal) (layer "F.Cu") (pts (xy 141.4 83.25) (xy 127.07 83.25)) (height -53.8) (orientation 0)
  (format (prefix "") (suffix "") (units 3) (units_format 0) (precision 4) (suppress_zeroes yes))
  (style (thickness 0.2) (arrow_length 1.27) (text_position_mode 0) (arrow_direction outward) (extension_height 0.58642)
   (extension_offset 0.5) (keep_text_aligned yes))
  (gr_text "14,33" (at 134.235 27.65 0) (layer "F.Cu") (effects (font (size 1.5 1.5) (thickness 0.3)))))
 (segment (start 173.3 143.75) (end 172.7 143.75) (width 0.2) (layer "F.Cu") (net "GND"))
 (via (at 172.7 143.75) (size 0.6) (drill 0.3) (layers "F.Cu" "B.Cu") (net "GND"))
 (segment (start 172.7 143.75) (end 171.65 143.75) (width 0.2) (layer "B.Cu") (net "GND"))
 (segment (start 169.68925 143.75) (end 169.67675 143.7625) (width 0.2) (layer "B.Cu") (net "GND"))
 (segment (start 171.65 143.75) (end 169.68925 143.75) (width 0.2) (layer "B.Cu") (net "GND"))
 (segment (start 173.3 145.35) (end 173.1 145.35) (width 0.2) (layer "F.Cu") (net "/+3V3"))
 (segment (start 173.1 145.35) (end 172.6 145.85) (width 0.2) (layer "F.Cu") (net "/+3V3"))
 (segment (start 139.1125 56.575) (end 138.7875 56.25) (width 0.2) (layer "F.Cu") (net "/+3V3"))
 (via (at 172.6 145.85) (size 0.6) (drill 0.3) (layers "F.Cu" "B.Cu") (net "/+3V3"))
 (segment (start 171.65 145.825) (end 169.68925 145.825) (width 0.2) (layer "B.Cu") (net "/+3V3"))
 (segment (start 171.675 145.85) (end 171.65 145.825) (width 0.2) (layer "B.Cu") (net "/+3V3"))
 (segment (start 169.68925 145.825) (end 169.67675 145.8375) (width 0.2) (layer "B.Cu") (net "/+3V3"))
 (segment (start 172.6 145.85) (end 171.675 145.85) (width 0.2) (layer "B.Cu") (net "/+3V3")))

